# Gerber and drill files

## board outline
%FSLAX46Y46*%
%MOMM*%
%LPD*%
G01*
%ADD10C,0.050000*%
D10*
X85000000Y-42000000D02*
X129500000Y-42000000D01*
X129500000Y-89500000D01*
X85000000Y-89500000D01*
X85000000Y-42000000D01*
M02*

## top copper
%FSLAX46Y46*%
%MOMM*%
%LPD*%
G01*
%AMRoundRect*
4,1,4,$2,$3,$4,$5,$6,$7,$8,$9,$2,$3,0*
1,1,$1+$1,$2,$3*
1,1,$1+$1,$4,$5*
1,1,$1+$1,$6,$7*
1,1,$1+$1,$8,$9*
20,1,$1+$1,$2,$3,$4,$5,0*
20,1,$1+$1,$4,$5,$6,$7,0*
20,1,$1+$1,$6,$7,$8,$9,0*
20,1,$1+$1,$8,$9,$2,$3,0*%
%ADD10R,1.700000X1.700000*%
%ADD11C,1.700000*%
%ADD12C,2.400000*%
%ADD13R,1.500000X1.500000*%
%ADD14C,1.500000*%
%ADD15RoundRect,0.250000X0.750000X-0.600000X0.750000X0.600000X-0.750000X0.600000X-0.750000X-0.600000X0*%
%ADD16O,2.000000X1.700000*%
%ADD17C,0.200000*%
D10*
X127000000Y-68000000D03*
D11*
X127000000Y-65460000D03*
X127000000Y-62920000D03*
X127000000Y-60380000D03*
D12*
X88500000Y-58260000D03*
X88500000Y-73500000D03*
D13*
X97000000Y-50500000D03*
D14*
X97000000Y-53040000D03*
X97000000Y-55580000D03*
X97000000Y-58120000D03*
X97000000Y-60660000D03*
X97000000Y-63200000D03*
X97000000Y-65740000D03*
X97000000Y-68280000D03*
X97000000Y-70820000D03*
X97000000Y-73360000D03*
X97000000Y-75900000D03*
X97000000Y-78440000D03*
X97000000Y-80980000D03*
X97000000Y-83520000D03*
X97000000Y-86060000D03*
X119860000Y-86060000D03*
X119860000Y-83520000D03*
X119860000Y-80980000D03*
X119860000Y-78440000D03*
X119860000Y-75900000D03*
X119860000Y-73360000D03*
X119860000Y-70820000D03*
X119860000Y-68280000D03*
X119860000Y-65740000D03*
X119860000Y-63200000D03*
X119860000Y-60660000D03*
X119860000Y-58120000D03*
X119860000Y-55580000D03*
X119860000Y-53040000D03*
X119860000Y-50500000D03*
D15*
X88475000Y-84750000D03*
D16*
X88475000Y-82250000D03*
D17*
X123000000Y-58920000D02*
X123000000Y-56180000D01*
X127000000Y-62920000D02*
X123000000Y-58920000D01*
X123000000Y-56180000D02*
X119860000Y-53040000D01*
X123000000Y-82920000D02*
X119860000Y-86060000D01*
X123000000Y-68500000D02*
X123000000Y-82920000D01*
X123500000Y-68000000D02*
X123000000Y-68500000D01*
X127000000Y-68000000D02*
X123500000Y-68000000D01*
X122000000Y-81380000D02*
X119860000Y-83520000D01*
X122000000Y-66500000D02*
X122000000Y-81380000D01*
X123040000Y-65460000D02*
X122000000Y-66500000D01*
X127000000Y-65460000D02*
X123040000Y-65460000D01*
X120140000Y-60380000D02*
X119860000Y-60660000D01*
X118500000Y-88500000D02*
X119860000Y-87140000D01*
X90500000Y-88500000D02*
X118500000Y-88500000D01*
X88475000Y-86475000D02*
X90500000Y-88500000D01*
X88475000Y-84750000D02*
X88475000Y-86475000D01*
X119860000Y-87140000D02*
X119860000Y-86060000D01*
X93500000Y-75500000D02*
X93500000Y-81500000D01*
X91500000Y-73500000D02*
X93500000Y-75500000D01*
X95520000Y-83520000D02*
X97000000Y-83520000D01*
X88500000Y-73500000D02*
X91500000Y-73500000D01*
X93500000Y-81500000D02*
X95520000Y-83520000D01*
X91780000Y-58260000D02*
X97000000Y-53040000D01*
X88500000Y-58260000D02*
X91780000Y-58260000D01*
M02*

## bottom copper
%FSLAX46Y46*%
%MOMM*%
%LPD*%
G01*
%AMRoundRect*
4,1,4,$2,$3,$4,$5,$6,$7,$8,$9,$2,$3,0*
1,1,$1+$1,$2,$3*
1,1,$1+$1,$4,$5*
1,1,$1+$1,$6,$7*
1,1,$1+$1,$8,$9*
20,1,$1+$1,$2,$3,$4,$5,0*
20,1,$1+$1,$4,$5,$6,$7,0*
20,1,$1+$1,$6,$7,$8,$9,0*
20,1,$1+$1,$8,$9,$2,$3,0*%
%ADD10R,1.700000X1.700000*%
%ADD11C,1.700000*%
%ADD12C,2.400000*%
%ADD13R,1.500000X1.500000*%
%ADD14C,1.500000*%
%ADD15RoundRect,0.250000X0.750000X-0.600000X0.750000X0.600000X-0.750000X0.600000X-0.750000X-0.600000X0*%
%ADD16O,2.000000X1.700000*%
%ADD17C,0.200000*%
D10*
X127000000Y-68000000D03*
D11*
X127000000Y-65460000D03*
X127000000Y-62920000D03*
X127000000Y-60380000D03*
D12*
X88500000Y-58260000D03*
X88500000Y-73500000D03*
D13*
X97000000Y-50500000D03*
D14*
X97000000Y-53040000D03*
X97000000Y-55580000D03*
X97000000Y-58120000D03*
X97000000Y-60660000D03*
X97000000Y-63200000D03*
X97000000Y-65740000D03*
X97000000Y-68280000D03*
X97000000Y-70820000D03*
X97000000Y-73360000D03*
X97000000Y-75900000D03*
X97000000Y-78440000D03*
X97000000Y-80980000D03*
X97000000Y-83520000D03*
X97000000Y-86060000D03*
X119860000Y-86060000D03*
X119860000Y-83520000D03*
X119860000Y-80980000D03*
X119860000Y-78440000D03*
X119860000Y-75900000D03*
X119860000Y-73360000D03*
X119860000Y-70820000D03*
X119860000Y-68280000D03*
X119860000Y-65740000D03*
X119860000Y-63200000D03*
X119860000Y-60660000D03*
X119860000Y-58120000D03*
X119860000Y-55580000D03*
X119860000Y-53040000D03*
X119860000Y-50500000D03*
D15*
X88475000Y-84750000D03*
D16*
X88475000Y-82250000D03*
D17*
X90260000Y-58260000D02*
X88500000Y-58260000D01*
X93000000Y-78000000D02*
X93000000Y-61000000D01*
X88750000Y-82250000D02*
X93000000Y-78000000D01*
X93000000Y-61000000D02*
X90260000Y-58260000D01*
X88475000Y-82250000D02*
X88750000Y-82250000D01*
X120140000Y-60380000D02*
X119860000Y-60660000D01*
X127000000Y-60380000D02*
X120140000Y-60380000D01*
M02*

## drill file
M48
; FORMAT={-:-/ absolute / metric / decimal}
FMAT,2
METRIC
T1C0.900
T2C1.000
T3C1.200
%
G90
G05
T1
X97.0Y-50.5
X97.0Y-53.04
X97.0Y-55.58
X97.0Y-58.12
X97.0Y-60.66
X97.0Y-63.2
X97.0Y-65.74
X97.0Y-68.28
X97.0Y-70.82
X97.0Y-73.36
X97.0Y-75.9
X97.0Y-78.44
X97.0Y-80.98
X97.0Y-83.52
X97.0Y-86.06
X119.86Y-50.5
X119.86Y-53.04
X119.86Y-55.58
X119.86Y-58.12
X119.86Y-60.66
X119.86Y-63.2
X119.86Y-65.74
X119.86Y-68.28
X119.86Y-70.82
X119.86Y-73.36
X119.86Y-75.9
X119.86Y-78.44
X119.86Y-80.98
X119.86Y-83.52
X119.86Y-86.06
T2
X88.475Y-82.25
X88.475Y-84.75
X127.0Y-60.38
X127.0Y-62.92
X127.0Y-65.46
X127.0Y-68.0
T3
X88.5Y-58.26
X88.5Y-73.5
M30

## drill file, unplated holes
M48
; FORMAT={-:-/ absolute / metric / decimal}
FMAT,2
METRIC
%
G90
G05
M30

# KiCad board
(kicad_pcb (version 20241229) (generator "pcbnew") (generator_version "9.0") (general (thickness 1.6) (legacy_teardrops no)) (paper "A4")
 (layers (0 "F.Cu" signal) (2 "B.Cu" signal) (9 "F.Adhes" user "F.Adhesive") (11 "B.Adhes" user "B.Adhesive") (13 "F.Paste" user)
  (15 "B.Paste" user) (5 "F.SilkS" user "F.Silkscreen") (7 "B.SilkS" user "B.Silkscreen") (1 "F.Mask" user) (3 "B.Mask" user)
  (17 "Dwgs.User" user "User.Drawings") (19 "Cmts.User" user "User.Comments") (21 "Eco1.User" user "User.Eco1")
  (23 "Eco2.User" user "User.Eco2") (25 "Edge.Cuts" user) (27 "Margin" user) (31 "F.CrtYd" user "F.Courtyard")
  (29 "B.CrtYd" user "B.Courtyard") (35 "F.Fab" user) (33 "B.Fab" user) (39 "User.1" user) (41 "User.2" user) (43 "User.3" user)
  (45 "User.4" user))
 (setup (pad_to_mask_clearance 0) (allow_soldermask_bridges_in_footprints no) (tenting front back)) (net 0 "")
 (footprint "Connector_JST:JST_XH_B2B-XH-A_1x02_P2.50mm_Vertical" (layer "F.Cu") (at 88.475 84.75 90)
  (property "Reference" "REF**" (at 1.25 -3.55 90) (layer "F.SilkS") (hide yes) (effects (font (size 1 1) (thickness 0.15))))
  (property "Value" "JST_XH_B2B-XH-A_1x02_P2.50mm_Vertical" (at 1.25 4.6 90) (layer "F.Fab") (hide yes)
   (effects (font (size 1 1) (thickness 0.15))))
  (pad "1" thru_hole roundrect (at 0 0 90) (size 1.7 2) (drill 1) (layers "*.Cu" "*.Mask") (remove_unused_layers no)
   (roundrect_rratio 0.147059))
  (pad "2" thru_hole oval (at 2.5 0 90) (size 1.7 2) (drill 1) (layers "*.Cu" "*.Mask") (remove_unused_layers no)))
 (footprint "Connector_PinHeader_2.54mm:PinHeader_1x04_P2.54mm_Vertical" (layer "F.Cu") (at 127 68 180)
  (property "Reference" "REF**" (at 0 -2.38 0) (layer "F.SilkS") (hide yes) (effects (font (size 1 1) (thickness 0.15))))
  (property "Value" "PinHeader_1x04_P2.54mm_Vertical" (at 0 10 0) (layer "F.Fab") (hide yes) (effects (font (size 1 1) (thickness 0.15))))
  (pad "1" thru_hole rect (at 0 0 180) (size 1.7 1.7) (drill 1) (layers "*.Cu" "*.Mask") (remove_unused_layers no))
  (pad "2" thru_hole circle (at 0 2.54 180) (size 1.7 1.7) (drill 1) (layers "*.Cu" "*.Mask") (remove_unused_layers no))
  (pad "3" thru_hole circle (at 0 5.08 180) (size 1.7 1.7) (drill 1) (layers "*.Cu" "*.Mask") (remove_unused_layers no))
  (pad "4" thru_hole circle (at 0 7.62 180) (size 1.7 1.7) (drill 1) (layers "*.Cu" "*.Mask") (remove_unused_layers no)))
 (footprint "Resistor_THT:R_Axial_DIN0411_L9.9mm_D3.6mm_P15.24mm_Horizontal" (layer "F.Cu") (at 88.5 73.5 90)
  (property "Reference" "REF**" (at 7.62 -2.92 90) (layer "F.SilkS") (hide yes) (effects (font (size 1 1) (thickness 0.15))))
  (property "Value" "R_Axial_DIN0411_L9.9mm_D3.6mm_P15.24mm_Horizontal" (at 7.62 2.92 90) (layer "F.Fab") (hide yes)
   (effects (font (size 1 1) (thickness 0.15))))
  (pad "1" thru_hole circle (at 0 0 90) (size 2.4 2.4) (drill 1.2) (layers "*.Cu" "*.Mask") (remove_unused_layers no))
  (pad "2" thru_hole circle (at 15.24 0 90) (size 2.4 2.4) (drill 1.2) (layers "*.Cu" "*.Mask") (remove_unused_layers no)))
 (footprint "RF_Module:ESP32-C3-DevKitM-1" (layer "F.Cu") (at 97 50.5)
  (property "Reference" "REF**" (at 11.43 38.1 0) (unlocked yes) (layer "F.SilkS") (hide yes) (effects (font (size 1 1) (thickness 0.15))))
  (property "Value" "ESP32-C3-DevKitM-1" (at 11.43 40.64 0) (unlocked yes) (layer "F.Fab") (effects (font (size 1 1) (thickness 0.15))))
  (pad "1" thru_hole rect (at 0 0) (size 1.5 1.5) (drill 0.9) (layers "*.Cu" "*.Mask") (remove_unused_layers yes) (keep_end_layers yes)
   (zone_layer_connections))
  (pad "2" thru_hole circle (at 0 2.54) (size 1.5 1.5) (drill 0.9) (layers "*.Cu" "*.Mask") (remove_unused_layers yes) (keep_end_layers yes)
   (zone_layer_connections))
  (pad "3" thru_hole circle (at 0 5.08) (size 1.5 1.5) (drill 0.9) (layers "*.Cu" "*.Mask") (remove_unused_layers yes) (keep_end_layers yes)
   (zone_layer_connections))
  (pad "4" thru_hole circle (at 0 7.62) (size 1.5 1.5) (drill 0.9) (layers "*.Cu" "*.Mask") (remove_unused_layers yes) (keep_end_layers yes)
   (zone_layer_connections))
  (pad "5" thru_hole circle (at 0 10.16) (size 1.5 1.5) (drill 0.9) (layers "*.Cu" "*.Mask") (remove_unused_layers yes)
   (keep_end_layers yes) (zone_layer_connections))
  (pad "6" thru_hole circle (at 0 12.7) (size 1.5 1.5) (drill 0.9) (layers "*.Cu" "*.Mask") (remove_unused_layers yes) (keep_end_layers yes)
   (zone_layer_connections))
  (pad "7" thru_hole circle (at 0 15.24) (size 1.5 1.5) (drill 0.9) (layers "*.Cu" "*.Mask") (remove_unused_layers yes)
   (keep_end_layers yes) (zone_layer_connections))
  (pad "8" thru_hole circle (at 0 17.78) (size 1.5 1.5) (drill 0.9) (layers "*.Cu" "*.Mask") (remove_unused_layers yes)
   (keep_end_layers yes) (zone_layer_connections))
  (pad "9" thru_hole circle (at 0 20.32) (size 1.5 1.5) (drill 0.9) (layers "*.Cu" "*.Mask") (remove_unused_layers yes)
   (keep_end_layers yes) (zone_layer_connections))
  (pad "10" thru_hole circle (at 0 22.86) (size 1.5 1.5) (drill 0.9) (layers "*.Cu" "*.Mask") (remove_unused_layers yes)
   (keep_end_layers yes) (zone_layer_connections))
  (pad "11" thru_hole circle (at 0 25.4) (size 1.5 1.5) (drill 0.9) (layers "*.Cu" "*.Mask") (remove_unused_layers yes)
   (keep_end_layers yes) (zone_layer_connections))
  (pad "12" thru_hole circle (at 0 27.94) (size 1.5 1.5) (drill 0.9) (layers "*.Cu" "*.Mask") (remove_unused_layers yes)
   (keep_end_layers yes) (zone_layer_connections))
  (pad "13" thru_hole circle (at 0 30.48) (size 1.5 1.5) (drill 0.9) (layers "*.Cu" "*.Mask") (remove_unused_layers yes)
   (keep_end_layers yes) (zone_layer_connections))
  (pad "14" thru_hole circle (at 0 33.02) (size 1.5 1.5) (drill 0.9) (layers "*.Cu" "*.Mask") (remove_unused_layers yes)
   (keep_end_layers yes) (zone_layer_connections))
  (pad "15" thru_hole circle (at 0 35.56) (size 1.5 1.5) (drill 0.9) (layers "*.Cu" "*.Mask") (remove_unused_layers yes)
   (keep_end_layers yes) (zone_layer_connections))
  (pad "16" thru_hole circle (at 22.86 35.56) (size 1.5 1.5) (drill 0.9) (layers "*.Cu" "*.Mask") (remove_unused_layers yes)
   (keep_end_layers yes) (zone_layer_connections))
  (pad "17" thru_hole circle (at 22.86 33.02) (size 1.5 1.5) (drill 0.9) (layers "*.Cu" "*.Mask") (remove_unused_layers yes)
   (keep_end_layers yes) (zone_layer_connections))
  (pad "18" thru_hole circle (at 22.86 30.48) (size 1.5 1.5) (drill 0.9) (layers "*.Cu" "*.Mask") (remove_unused_layers yes)
   (keep_end_layers yes) (zone_layer_connections))
  (pad "19" thru_hole circle (at 22.86 27.94) (size 1.5 1.5) (drill 0.9) (layers "*.Cu" "*.Mask") (remove_unused_layers yes)
   (keep_end_layers yes) (zone_layer_connections))
  (pad "20" thru_hole circle (at 22.86 25.4) (size 1.5 1.5) (drill 0.9) (layers "*.Cu" "*.Mask") (remove_unused_layers yes)
   (keep_end_layers yes) (zone_layer_connections))
  (pad "21" thru_hole circle (at 22.86 22.86) (size 1.5 1.5) (drill 0.9) (layers "*.Cu" "*.Mask") (remove_unused_layers yes)
   (keep_end_layers yes) (zone_layer_connections))
  (pad "22" thru_hole circle (at 22.86 20.32) (size 1.5 1.5) (drill 0.9) (layers "*.Cu" "*.Mask") (remove_unused_layers yes)
   (keep_end_layers yes) (zone_layer_connections))
  (pad "23" thru_hole circle (at 22.86 17.78) (size 1.5 1.5) (drill 0.9) (layers "*.Cu" "*.Mask") (remove_unused_layers yes)
   (keep_end_layers yes) (zone_layer_connections))
  (pad "24" thru_hole circle (at 22.86 15.24) (size 1.5 1.5) (drill 0.9) (layers "*.Cu" "*.Mask") (remove_unused_layers yes)
   (keep_end_layers yes) (zone_layer_connections))
  (pad "25" thru_hole circle (at 22.86 12.7) (size 1.5 1.5) (drill 0.9) (layers "*.Cu" "*.Mask") (remove_unused_layers yes)
   (keep_end_layers yes) (zone_layer_connections))
  (pad "26" thru_hole circle (at 22.86 10.16) (size 1.5 1.5) (drill 0.9) (layers "*.Cu" "*.Mask") (remove_unused_layers yes)
   (keep_end_layers yes) (zone_layer_connections))
  (pad "27" thru_hole circle (at 22.86 7.62) (size 1.5 1.5) (drill 0.9) (layers "*.Cu" "*.Mask") (remove_unused_layers yes)
   (keep_end_layers yes) (zone_layer_connections))
  (pad "28" thru_hole circle (at 22.86 5.08) (size 1.5 1.5) (drill 0.9) (layers "*.Cu" "*.Mask") (remove_unused_layers yes)
   (keep_end_layers yes) (zone_layer_connections))
  (pad "29" thru_hole circle (at 22.86 2.54) (size 1.5 1.5) (drill 0.9) (layers "*.Cu" "*.Mask") (remove_unused_layers yes)
   (keep_end_layers yes) (zone_layer_connections))
  (pad "30" thru_hole circle (at 22.86 0) (size 1.5 1.5) (drill 0.9) (layers "*.Cu" "*.Mask") (remove_unused_layers yes)
   (keep_end_layers yes) (zone_layer_connections)))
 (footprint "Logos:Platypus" (layer "B.Cu") (at 102.5 62.5 180)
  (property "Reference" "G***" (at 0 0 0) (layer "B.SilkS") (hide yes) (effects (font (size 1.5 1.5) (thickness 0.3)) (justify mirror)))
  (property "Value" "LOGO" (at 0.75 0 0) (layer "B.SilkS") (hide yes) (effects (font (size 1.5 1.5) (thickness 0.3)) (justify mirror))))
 (gr_rect (start 85 42) (end 129.5 89.5) (stroke (width 0.05) (type default)) (fill no) (layer "Edge.Cuts"))
 (segment (start 88.5 73.5) (end 91.5 73.5) (width 0.2) (layer "F.Cu") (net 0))
 (segment (start 95.52 83.52) (end 97 83.52) (width 0.2) (layer "F.Cu") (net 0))
 (segment (start 88.475 86.475) (end 90.5 88.5) (width 0.2) (layer "F.Cu") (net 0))
 (segment (start 93.5 75.5) (end 93.5 81.5) (width 0.2) (layer "F.Cu") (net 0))
 (segment (start 123 82.92) (end 119.86 86.06) (width 0.2) (layer "F.Cu") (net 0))
 (segment (start 88.5 58.26) (end 91.78 58.26) (width 0.2) (layer "F.Cu") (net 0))
 (segment (start 118.5 88.5) (end 119.86 87.14) (width 0.2) (layer "F.Cu") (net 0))
 (segment (start 123 58.92) (end 123 56.18) (width 0.2) (layer "F.Cu") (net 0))
 (segment (start 127 62.92) (end 123 58.92) (width 0.2) (layer "F.Cu") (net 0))
 (segment (start 123 68.5) (end 123 82.92) (width 0.2) (layer "F.Cu") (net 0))
 (segment (start 119.86 87.14) (end 119.86 86.06) (width 0.2) (layer "F.Cu") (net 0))
 (segment (start 91.78 58.26) (end 97 53.04) (width 0.2) (layer "F.Cu") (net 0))
 (segment (start 123.04 65.46) (end 122 66.5) (width 0.2) (layer "F.Cu") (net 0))
 (segment (start 93.5 81.5) (end 95.52 83.52) (width 0.2) (layer "F.Cu") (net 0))
 (segment (start 122 81.38) (end 119.86 83.52) (width 0.2) (layer "F.Cu") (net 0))
 (segment (start 90.5 88.5) (end 118.5 88.5) (width 0.2) (layer "F.Cu") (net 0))
 (segment (start 122 66.5) (end 122 81.38) (width 0.2) (layer "F.Cu") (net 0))
 (segment (start 127 65.46) (end 123.04 65.46) (width 0.2) (layer "F.Cu") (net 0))
 (segment (start 123 56.18) (end 119.86 53.04) (width 0.2) (layer "F.Cu") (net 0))
 (segment (start 123.5 68) (end 123 68.5) (width 0.2) (layer "F.Cu") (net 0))
 (segment (start 88.475 84.75) (end 88.475 86.475) (width 0.2) (layer "F.Cu") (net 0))
 (segment (start 120.14 60.38) (end 119.86 60.66) (width 0.2) (layer "F.Cu") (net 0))
 (segment (start 91.5 73.5) (end 93.5 75.5) (width 0.2) (layer "F.Cu") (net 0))
 (segment (start 127 68) (end 123.5 68) (width 0.2) (layer "F.Cu") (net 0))
 (segment (start 90.26 58.26) (end 88.5 58.26) (width 0.2) (layer "B.Cu") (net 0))
 (segment (start 127 60.38) (end 120.14 60.38) (width 0.2) (layer "B.Cu") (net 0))
 (segment (start 88.75 82.25) (end 93 78) (width 0.2) (layer "B.Cu") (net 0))
 (segment (start 88.475 82.25) (end 88.75 82.25) (width 0.2) (layer "B.Cu") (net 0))
 (segment (start 93 78) (end 93 61) (width 0.2) (layer "B.Cu") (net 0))
 (segment (start 120.14 60.38) (end 119.86 60.66) (width 0.2) (layer "B.Cu") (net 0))
 (segment (start 93 61) (end 90.26 58.26) (width 0.2) (layer "B.Cu") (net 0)))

